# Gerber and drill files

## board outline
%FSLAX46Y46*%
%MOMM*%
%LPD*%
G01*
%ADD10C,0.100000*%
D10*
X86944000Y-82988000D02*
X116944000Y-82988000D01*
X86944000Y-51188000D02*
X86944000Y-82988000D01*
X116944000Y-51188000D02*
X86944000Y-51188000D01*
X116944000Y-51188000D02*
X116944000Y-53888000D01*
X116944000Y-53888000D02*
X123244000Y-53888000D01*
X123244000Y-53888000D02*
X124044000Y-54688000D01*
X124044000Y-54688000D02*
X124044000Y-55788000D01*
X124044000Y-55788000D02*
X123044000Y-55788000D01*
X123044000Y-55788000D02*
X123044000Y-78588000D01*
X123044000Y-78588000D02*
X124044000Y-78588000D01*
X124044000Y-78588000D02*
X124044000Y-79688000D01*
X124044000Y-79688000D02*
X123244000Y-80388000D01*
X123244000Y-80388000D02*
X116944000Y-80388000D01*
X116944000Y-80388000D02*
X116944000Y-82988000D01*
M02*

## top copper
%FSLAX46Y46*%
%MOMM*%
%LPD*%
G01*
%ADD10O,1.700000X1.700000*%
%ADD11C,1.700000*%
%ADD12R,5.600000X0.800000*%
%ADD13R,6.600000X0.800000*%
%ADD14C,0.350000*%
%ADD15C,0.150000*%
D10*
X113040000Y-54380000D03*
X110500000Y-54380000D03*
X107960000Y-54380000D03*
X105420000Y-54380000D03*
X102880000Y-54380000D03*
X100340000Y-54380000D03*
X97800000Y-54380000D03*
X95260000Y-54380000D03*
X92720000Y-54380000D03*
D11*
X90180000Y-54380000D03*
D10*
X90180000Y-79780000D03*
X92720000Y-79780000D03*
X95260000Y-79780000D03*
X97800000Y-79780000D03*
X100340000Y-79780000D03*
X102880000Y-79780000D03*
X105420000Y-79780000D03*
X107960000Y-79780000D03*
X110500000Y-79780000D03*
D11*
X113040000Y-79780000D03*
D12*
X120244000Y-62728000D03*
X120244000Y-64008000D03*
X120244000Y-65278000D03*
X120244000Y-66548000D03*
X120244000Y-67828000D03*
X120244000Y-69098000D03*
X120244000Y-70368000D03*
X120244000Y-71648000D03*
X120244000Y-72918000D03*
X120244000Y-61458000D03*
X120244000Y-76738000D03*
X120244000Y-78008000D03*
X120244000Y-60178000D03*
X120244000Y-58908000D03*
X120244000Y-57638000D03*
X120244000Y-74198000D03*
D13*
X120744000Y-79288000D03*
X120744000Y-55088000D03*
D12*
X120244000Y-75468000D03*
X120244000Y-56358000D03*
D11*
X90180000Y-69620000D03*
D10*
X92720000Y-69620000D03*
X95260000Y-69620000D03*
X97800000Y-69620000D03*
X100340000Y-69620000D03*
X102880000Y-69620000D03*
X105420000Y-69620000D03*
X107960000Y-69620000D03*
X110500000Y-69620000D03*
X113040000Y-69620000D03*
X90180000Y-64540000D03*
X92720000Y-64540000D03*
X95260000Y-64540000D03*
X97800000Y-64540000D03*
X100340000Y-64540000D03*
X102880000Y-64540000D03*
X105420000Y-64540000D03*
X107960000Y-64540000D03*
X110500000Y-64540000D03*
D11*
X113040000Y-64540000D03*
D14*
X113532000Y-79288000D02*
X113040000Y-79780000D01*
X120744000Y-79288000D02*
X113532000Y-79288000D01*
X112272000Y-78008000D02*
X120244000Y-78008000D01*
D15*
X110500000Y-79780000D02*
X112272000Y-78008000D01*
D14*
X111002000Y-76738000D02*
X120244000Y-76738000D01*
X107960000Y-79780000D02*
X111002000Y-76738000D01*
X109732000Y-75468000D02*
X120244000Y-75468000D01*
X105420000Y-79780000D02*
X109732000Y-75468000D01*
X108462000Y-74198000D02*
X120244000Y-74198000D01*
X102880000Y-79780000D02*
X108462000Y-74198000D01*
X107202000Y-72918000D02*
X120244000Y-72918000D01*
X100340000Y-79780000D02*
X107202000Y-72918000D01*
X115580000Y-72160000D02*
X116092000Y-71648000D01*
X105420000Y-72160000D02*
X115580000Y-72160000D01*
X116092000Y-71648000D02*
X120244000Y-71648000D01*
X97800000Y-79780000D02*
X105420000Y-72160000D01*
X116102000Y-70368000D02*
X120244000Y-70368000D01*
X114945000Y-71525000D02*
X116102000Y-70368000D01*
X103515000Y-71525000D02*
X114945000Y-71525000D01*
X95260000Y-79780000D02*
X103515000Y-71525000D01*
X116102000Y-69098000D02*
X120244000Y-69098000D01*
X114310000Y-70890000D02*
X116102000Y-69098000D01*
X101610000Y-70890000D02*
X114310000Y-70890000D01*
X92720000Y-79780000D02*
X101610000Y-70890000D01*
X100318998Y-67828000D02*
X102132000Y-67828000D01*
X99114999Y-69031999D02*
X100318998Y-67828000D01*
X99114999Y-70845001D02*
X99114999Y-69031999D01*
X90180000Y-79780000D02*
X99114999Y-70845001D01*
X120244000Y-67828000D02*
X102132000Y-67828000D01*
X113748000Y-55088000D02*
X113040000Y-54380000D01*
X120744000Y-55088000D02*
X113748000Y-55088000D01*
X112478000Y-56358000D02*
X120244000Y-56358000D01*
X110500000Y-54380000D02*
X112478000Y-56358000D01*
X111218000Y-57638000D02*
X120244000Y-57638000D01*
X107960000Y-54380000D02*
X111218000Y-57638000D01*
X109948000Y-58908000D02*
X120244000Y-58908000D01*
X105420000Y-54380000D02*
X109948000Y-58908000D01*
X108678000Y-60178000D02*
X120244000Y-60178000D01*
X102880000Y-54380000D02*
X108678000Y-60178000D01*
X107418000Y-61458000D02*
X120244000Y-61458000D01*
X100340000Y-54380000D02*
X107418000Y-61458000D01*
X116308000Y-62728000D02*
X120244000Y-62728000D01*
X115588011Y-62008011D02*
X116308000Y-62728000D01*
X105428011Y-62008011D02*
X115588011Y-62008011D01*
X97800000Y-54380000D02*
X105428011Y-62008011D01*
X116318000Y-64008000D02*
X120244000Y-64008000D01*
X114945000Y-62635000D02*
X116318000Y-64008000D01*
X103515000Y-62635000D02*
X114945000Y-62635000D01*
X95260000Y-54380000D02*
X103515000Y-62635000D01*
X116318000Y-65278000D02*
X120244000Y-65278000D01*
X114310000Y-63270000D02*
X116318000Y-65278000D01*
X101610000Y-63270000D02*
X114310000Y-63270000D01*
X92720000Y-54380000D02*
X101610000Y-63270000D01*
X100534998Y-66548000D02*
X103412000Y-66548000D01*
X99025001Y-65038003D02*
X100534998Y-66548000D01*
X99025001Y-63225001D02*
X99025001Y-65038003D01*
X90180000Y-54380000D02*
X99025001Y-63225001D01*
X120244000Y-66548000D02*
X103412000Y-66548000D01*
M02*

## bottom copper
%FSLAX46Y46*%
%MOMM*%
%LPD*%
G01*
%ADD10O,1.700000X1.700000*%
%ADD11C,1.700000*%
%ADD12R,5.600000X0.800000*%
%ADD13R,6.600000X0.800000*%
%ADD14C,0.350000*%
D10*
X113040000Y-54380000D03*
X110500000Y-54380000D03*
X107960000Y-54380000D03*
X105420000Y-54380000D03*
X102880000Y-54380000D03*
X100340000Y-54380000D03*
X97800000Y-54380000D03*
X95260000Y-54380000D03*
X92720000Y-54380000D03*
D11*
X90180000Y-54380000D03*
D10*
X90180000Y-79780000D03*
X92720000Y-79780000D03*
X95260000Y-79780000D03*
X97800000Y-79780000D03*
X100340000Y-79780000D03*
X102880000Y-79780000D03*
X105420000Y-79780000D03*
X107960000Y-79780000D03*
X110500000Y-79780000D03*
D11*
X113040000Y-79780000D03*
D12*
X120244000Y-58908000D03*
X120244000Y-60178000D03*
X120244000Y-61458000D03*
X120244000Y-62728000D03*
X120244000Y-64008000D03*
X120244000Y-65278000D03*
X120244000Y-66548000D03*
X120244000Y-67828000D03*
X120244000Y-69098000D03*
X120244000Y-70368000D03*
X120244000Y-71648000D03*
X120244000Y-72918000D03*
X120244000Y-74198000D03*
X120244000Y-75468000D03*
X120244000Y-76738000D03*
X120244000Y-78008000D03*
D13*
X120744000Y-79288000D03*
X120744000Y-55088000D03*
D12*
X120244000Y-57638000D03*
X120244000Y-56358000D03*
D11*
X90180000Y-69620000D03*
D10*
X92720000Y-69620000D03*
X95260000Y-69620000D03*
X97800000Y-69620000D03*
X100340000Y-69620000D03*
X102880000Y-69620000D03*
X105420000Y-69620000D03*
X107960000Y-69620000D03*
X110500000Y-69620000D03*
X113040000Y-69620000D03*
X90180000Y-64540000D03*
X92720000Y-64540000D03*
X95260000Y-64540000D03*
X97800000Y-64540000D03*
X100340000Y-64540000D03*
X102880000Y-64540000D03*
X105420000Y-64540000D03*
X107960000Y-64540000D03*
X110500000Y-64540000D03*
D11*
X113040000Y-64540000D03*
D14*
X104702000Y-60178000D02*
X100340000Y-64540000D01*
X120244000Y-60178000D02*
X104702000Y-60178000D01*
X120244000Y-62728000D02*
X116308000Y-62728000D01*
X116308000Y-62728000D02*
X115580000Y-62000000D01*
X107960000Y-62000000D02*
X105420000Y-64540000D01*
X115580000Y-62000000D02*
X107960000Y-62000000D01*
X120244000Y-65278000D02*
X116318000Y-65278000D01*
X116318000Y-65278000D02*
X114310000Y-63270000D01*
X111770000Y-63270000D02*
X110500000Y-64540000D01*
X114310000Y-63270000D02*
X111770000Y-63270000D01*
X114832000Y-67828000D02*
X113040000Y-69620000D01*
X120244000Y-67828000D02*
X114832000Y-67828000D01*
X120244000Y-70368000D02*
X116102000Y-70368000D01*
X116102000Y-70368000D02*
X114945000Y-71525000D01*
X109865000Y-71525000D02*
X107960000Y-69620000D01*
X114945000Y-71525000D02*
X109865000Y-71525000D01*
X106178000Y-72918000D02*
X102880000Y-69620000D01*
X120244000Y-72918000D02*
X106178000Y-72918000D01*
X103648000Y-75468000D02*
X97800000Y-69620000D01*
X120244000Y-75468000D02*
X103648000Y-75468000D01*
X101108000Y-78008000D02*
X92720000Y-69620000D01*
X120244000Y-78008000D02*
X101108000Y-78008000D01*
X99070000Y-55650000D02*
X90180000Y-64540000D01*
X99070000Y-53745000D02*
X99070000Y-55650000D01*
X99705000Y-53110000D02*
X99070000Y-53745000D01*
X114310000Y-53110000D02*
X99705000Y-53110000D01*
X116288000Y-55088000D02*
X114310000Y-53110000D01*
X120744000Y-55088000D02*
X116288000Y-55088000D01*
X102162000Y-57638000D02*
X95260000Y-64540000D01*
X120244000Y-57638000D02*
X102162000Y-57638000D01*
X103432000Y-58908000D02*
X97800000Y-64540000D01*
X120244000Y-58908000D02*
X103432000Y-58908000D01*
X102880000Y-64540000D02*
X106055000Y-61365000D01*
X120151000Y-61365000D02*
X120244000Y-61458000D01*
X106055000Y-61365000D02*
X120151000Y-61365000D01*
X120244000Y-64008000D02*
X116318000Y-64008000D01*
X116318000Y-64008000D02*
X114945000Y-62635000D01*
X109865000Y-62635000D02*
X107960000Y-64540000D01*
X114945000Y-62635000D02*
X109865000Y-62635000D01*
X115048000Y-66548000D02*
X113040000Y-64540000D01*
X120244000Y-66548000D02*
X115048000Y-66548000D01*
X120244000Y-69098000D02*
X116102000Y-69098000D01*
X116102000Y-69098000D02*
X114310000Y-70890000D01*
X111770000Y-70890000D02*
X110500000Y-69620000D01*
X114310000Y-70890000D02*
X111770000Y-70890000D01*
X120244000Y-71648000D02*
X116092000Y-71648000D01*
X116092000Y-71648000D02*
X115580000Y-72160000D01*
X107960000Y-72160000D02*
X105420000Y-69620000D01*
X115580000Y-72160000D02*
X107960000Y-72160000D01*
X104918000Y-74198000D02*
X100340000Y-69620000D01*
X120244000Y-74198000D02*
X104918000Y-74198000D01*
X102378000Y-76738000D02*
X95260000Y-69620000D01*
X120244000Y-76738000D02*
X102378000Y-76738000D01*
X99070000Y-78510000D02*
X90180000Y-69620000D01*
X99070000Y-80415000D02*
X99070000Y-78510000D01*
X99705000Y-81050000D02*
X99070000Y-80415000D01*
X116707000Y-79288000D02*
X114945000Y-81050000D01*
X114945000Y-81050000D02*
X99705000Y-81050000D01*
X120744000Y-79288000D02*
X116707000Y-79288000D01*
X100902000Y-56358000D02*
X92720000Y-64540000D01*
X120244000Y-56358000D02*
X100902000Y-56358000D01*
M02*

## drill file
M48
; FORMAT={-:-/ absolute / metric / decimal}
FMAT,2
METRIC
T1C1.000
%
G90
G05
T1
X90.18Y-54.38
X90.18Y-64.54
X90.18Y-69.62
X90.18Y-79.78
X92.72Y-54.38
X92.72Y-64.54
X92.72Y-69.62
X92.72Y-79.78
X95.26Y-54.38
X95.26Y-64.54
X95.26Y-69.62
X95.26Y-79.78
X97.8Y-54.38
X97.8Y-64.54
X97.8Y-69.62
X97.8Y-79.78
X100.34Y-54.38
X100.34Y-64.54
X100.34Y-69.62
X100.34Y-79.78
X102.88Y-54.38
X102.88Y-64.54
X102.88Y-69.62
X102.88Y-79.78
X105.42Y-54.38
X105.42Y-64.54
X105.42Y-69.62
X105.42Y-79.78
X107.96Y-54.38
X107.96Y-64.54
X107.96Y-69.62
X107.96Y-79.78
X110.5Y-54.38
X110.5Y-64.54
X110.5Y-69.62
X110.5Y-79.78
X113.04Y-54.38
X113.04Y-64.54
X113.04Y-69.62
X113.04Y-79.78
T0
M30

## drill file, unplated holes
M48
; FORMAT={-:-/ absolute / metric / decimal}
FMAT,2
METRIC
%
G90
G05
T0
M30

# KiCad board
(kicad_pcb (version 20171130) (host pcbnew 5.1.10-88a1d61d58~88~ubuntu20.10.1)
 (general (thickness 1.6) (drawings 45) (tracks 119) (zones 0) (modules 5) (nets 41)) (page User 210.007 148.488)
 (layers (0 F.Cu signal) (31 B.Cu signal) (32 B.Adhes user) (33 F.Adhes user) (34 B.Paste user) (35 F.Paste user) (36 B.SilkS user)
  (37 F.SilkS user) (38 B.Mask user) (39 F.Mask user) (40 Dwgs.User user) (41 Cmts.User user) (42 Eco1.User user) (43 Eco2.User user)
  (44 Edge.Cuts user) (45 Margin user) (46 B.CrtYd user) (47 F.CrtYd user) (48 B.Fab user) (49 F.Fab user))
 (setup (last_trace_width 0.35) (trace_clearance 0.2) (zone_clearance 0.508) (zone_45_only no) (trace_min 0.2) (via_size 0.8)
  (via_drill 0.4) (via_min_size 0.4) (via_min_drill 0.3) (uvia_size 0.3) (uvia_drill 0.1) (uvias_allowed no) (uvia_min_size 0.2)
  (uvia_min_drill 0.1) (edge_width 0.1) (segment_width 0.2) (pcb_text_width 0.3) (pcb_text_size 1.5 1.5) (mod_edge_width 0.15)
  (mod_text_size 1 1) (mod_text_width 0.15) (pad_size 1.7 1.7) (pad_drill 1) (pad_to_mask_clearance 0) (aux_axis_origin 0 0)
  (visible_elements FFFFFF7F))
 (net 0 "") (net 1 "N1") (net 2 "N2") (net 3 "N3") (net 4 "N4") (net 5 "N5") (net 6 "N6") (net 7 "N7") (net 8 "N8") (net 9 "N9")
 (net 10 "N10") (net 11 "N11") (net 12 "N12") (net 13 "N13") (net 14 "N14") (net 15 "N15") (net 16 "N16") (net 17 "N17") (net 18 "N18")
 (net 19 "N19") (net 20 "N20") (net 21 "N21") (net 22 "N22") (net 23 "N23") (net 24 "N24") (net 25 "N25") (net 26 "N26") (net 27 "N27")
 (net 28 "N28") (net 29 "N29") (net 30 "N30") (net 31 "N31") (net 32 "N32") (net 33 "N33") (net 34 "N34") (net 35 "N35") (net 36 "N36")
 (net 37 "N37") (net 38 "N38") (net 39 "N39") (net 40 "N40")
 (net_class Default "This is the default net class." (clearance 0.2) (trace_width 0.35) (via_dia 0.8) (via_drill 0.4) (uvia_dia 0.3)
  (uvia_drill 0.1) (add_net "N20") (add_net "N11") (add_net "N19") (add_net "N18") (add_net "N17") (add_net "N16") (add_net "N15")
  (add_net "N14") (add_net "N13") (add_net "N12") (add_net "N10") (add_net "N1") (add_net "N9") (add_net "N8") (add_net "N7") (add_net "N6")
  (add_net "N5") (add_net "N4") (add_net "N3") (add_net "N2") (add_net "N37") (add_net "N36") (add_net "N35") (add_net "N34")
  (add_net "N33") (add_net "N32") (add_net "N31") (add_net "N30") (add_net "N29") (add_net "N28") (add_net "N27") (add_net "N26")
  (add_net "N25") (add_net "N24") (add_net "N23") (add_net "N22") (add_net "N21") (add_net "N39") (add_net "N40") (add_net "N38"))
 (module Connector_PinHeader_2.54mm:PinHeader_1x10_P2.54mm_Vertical (layer F.Cu) (at 90.18 54.38 90)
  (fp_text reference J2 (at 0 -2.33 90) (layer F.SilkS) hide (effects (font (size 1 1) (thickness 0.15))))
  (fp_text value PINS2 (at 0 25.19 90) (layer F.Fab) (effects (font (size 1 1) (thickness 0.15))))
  (pad 10 thru_hole oval (at 0 22.86 90) (size 1.7 1.7) (drill 1) (layers *.Cu *.Mask) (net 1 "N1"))
  (pad 9 thru_hole oval (at 0 20.32 90) (size 1.7 1.7) (drill 1) (layers *.Cu *.Mask) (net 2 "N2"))
  (pad 8 thru_hole oval (at 0 17.78 90) (size 1.7 1.7) (drill 1) (layers *.Cu *.Mask) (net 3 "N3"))
  (pad 7 thru_hole oval (at 0 15.24 90) (size 1.7 1.7) (drill 1) (layers *.Cu *.Mask) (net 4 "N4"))
  (pad 6 thru_hole oval (at 0 12.7 90) (size 1.7 1.7) (drill 1) (layers *.Cu *.Mask) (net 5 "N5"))
  (pad 5 thru_hole oval (at 0 10.16 90) (size 1.7 1.7) (drill 1) (layers *.Cu *.Mask) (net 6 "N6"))
  (pad 4 thru_hole oval (at 0 7.62 90) (size 1.7 1.7) (drill 1) (layers *.Cu *.Mask) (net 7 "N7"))
  (pad 3 thru_hole oval (at 0 5.08 90) (size 1.7 1.7) (drill 1) (layers *.Cu *.Mask) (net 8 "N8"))
  (pad 2 thru_hole oval (at 0 2.54 90) (size 1.7 1.7) (drill 1) (layers *.Cu *.Mask) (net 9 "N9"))
  (pad 1 thru_hole circle (at 0 0 90) (size 1.7 1.7) (drill 1) (layers *.Cu *.Mask) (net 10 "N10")))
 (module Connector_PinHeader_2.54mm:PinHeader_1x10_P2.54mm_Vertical (layer F.Cu) (at 113.04 79.78 270)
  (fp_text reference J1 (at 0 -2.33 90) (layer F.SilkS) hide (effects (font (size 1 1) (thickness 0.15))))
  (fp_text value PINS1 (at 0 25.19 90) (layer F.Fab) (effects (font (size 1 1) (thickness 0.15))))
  (pad 10 thru_hole oval (at 0 22.86 270) (size 1.7 1.7) (drill 1) (layers *.Cu *.Mask) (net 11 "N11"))
  (pad 9 thru_hole oval (at 0 20.32 270) (size 1.7 1.7) (drill 1) (layers *.Cu *.Mask) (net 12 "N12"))
  (pad 8 thru_hole oval (at 0 17.78 270) (size 1.7 1.7) (drill 1) (layers *.Cu *.Mask) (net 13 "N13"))
  (pad 7 thru_hole oval (at 0 15.24 270) (size 1.7 1.7) (drill 1) (layers *.Cu *.Mask) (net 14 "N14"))
  (pad 6 thru_hole oval (at 0 12.7 270) (size 1.7 1.7) (drill 1) (layers *.Cu *.Mask) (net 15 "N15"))
  (pad 5 thru_hole oval (at 0 10.16 270) (size 1.7 1.7) (drill 1) (layers *.Cu *.Mask) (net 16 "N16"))
  (pad 4 thru_hole oval (at 0 7.62 270) (size 1.7 1.7) (drill 1) (layers *.Cu *.Mask) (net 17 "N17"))
  (pad 3 thru_hole oval (at 0 5.08 270) (size 1.7 1.7) (drill 1) (layers *.Cu *.Mask) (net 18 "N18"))
  (pad 2 thru_hole oval (at 0 2.54 270) (size 1.7 1.7) (drill 1) (layers *.Cu *.Mask) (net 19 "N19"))
  (pad 1 thru_hole circle (at 0 0 270) (size 1.7 1.7) (drill 1) (layers *.Cu *.Mask) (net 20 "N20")))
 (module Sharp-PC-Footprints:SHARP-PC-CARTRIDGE (layer F.Cu) (at 116.944 51.188)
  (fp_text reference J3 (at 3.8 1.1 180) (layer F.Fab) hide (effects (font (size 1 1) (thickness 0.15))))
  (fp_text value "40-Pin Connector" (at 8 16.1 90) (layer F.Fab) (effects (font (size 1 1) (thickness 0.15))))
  (fp_line (start 0 0) (end 0 2.7) (layer Edge.Cuts) (width 0.1))
  (fp_line (start 0 2.7) (end 6.3 2.7) (layer Edge.Cuts) (width 0.1))
  (fp_line (start 6.3 2.7) (end 7.1 3.5) (layer Edge.Cuts) (width 0.1))
  (fp_line (start 7.1 3.5) (end 7.1 4.6) (layer Edge.Cuts) (width 0.1))
  (fp_line (start 7.1 4.6) (end 6.1 4.6) (layer Edge.Cuts) (width 0.1))
  (fp_line (start 6.1 4.6) (end 6.1 27.4) (layer Edge.Cuts) (width 0.1))
  (fp_line (start 6.1 27.4) (end 7.1 27.4) (layer Edge.Cuts) (width 0.1))
  (fp_line (start 7.1 27.4) (end 7.1 28.5) (layer Edge.Cuts) (width 0.1))
  (fp_line (start 7.1 28.5) (end 6.3 29.2) (layer Edge.Cuts) (width 0.1))
  (fp_line (start 6.3 29.2) (end 0 29.2) (layer Edge.Cuts) (width 0.1))
  (fp_line (start 0 29.2) (end 0 31.8) (layer Edge.Cuts) (width 0.1))
  (pad 37 smd rect (at 3.3 7.72 180) (size 5.6 0.8) (layers B.Cu B.Paste B.Mask) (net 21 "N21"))
  (pad 36 smd rect (at 3.3 8.99 180) (size 5.6 0.8) (layers B.Cu B.Paste B.Mask) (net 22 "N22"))
  (pad 35 smd rect (at 3.3 10.27 180) (size 5.6 0.8) (layers B.Cu B.Paste B.Mask) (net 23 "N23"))
  (pad 34 smd rect (at 3.3 11.54 180) (size 5.6 0.8) (layers B.Cu B.Paste B.Mask) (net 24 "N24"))
  (pad 33 smd rect (at 3.3 12.82 180) (size 5.6 0.8) (layers B.Cu B.Paste B.Mask) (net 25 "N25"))
  (pad 32 smd rect (at 3.3 14.09 180) (size 5.6 0.8) (layers B.Cu B.Paste B.Mask) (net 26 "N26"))
  (pad 31 smd rect (at 3.3 15.36 180) (size 5.6 0.8) (layers B.Cu B.Paste B.Mask) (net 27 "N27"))
  (pad 30 smd rect (at 3.3 16.64 180) (size 5.6 0.8) (layers B.Cu B.Paste B.Mask) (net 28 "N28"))
  (pad 29 smd rect (at 3.3 17.91 180) (size 5.6 0.8) (layers B.Cu B.Paste B.Mask) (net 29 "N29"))
  (pad 28 smd rect (at 3.3 19.18 180) (size 5.6 0.8) (layers B.Cu B.Paste B.Mask) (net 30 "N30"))
  (pad 27 smd rect (at 3.3 20.46 180) (size 5.6 0.8) (layers B.Cu B.Paste B.Mask) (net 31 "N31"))
  (pad 26 smd rect (at 3.3 21.73 180) (size 5.6 0.8) (layers B.Cu B.Paste B.Mask) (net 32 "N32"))
  (pad 25 smd rect (at 3.3 23.01 180) (size 5.6 0.8) (layers B.Cu B.Paste B.Mask) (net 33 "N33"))
  (pad 24 smd rect (at 3.3 24.28 180) (size 5.6 0.8) (layers B.Cu B.Paste B.Mask) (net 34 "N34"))
  (pad 23 smd rect (at 3.3 25.55 180) (size 5.6 0.8) (layers B.Cu B.Paste B.Mask) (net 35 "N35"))
  (pad 22 smd rect (at 3.3 26.82 180) (size 5.6 0.8) (layers B.Cu B.Paste B.Mask) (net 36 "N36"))
  (pad 14 smd rect (at 3.3 11.54 180) (size 5.6 0.8) (layers F.Cu F.Paste F.Mask) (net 7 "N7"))
  (pad 13 smd rect (at 3.3 12.82 180) (size 5.6 0.8) (layers F.Cu F.Paste F.Mask) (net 8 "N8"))
  (pad 12 smd rect (at 3.3 14.09 180) (size 5.6 0.8) (layers F.Cu F.Paste F.Mask) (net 9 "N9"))
  (pad 11 smd rect (at 3.3 15.36 180) (size 5.6 0.8) (layers F.Cu F.Paste F.Mask) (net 10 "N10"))
  (pad 10 smd rect (at 3.3 16.64 180) (size 5.6 0.8) (layers F.Cu F.Paste F.Mask) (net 11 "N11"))
  (pad 9 smd rect (at 3.3 17.91 180) (size 5.6 0.8) (layers F.Cu F.Paste F.Mask) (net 12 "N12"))
  (pad 8 smd rect (at 3.3 19.18 180) (size 5.6 0.8) (layers F.Cu F.Paste F.Mask) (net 13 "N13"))
  (pad 7 smd rect (at 3.3 20.46 180) (size 5.6 0.8) (layers F.Cu F.Paste F.Mask) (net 14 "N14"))
  (pad 6 smd rect (at 3.3 21.73 180) (size 5.6 0.8) (layers F.Cu F.Paste F.Mask) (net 15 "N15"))
  (pad 21 smd rect (at 3.8 28.1 180) (size 6.6 0.8) (layers B.Cu B.Paste B.Mask) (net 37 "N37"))
  (pad 40 smd rect (at 3.8 3.9 180) (size 6.6 0.8) (layers B.Cu B.Paste B.Mask) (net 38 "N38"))
  (pad 15 smd rect (at 3.3 10.27 180) (size 5.6 0.8) (layers F.Cu F.Paste F.Mask) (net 6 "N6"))
  (pad 38 smd rect (at 3.3 6.45 180) (size 5.6 0.8) (layers B.Cu B.Paste B.Mask) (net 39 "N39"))
  (pad 3 smd rect (at 3.3 25.55 180) (size 5.6 0.8) (layers F.Cu F.Paste F.Mask) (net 18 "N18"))
  (pad 2 smd rect (at 3.3 26.82 180) (size 5.6 0.8) (layers F.Cu F.Paste F.Mask) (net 19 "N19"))
  (pad 39 smd rect (at 3.3 5.17 180) (size 5.6 0.8) (layers B.Cu B.Paste B.Mask) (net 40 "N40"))
  (pad 16 smd rect (at 3.3 8.99 180) (size 5.6 0.8) (layers F.Cu F.Paste F.Mask) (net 5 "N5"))
  (pad 17 smd rect (at 3.3 7.72 180) (size 5.6 0.8) (layers F.Cu F.Paste F.Mask) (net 4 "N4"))
  (pad 18 smd rect (at 3.3 6.45 180) (size 5.6 0.8) (layers F.Cu F.Paste F.Mask) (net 3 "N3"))
  (pad 5 smd rect (at 3.3 23.01 180) (size 5.6 0.8) (layers F.Cu F.Paste F.Mask) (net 16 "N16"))
  (pad 1 smd rect (at 3.8 28.1 180) (size 6.6 0.8) (layers F.Cu F.Paste F.Mask) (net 20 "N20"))
  (pad 20 smd rect (at 3.8 3.9 180) (size 6.6 0.8) (layers F.Cu F.Paste F.Mask) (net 1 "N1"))
  (pad 4 smd rect (at 3.3 24.28 180) (size 5.6 0.8) (layers F.Cu F.Paste F.Mask) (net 17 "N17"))
  (pad 19 smd rect (at 3.3 5.17 180) (size 5.6 0.8) (layers F.Cu F.Paste F.Mask) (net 2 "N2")))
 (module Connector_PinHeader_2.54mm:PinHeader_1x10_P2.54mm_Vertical (layer F.Cu) (at 90.18 69.62 90)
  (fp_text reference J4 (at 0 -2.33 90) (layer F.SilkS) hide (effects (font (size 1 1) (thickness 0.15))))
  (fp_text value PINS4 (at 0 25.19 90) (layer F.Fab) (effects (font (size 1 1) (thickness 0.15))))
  (pad 1 thru_hole circle (at 0 0 90) (size 1.7 1.7) (drill 1) (layers *.Cu *.Mask) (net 37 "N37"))
  (pad 2 thru_hole oval (at 0 2.54 90) (size 1.7 1.7) (drill 1) (layers *.Cu *.Mask) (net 36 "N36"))
  (pad 3 thru_hole oval (at 0 5.08 90) (size 1.7 1.7) (drill 1) (layers *.Cu *.Mask) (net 35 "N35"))
  (pad 4 thru_hole oval (at 0 7.62 90) (size 1.7 1.7) (drill 1) (layers *.Cu *.Mask) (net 34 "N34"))
  (pad 5 thru_hole oval (at 0 10.16 90) (size 1.7 1.7) (drill 1) (layers *.Cu *.Mask) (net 33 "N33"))
  (pad 6 thru_hole oval (at 0 12.7 90) (size 1.7 1.7) (drill 1) (layers *.Cu *.Mask) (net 32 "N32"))
  (pad 7 thru_hole oval (at 0 15.24 90) (size 1.7 1.7) (drill 1) (layers *.Cu *.Mask) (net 31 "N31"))
  (pad 8 thru_hole oval (at 0 17.78 90) (size 1.7 1.7) (drill 1) (layers *.Cu *.Mask) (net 30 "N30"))
  (pad 9 thru_hole oval (at 0 20.32 90) (size 1.7 1.7) (drill 1) (layers *.Cu *.Mask) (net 29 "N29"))
  (pad 10 thru_hole oval (at 0 22.86 90) (size 1.7 1.7) (drill 1) (layers *.Cu *.Mask) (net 28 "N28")))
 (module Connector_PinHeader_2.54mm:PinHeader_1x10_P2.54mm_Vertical (layer F.Cu) (at 113.04 64.54 270)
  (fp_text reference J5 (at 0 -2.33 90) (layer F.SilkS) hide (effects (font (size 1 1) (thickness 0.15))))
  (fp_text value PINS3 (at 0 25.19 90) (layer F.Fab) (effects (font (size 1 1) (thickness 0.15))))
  (pad 10 thru_hole oval (at 0 22.86 270) (size 1.7 1.7) (drill 1) (layers *.Cu *.Mask) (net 38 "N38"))
  (pad 9 thru_hole oval (at 0 20.32 270) (size 1.7 1.7) (drill 1) (layers *.Cu *.Mask) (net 40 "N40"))
  (pad 8 thru_hole oval (at 0 17.78 270) (size 1.7 1.7) (drill 1) (layers *.Cu *.Mask) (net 39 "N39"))
  (pad 7 thru_hole oval (at 0 15.24 270) (size 1.7 1.7) (drill 1) (layers *.Cu *.Mask) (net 21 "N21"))
  (pad 6 thru_hole oval (at 0 12.7 270) (size 1.7 1.7) (drill 1) (layers *.Cu *.Mask) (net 22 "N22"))
  (pad 5 thru_hole oval (at 0 10.16 270) (size 1.7 1.7) (drill 1) (layers *.Cu *.Mask) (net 23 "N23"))
  (pad 4 thru_hole oval (at 0 7.62 270) (size 1.7 1.7) (drill 1) (layers *.Cu *.Mask) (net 24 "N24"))
  (pad 3 thru_hole oval (at 0 5.08 270) (size 1.7 1.7) (drill 1) (layers *.Cu *.Mask) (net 25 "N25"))
  (pad 2 thru_hole oval (at 0 2.54 270) (size 1.7 1.7) (drill 1) (layers *.Cu *.Mask) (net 26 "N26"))
  (pad 1 thru_hole circle (at 0 0 270) (size 1.7 1.7) (drill 1) (layers *.Cu *.Mask) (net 27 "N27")))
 (gr_line (start 86.944 82.988) (end 116.944 82.988) (layer Edge.Cuts) (width 0.1))
 (gr_line (start 86.944 51.188) (end 86.944 82.988) (layer Edge.Cuts) (width 0.1))
 (gr_line (start 116.944 51.188) (end 86.944 51.188) (layer Edge.Cuts) (width 0.1))
 (segment (start 113.532 79.288) (end 113.04 79.78) (width 0.35) (layer F.Cu) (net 20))
 (segment (start 120.744 79.288) (end 113.532 79.288) (width 0.35) (layer F.Cu) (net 20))
 (segment (start 112.272 78.008) (end 120.244 78.008) (width 0.35) (layer F.Cu) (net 19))
 (segment (start 110.5 79.78) (end 112.272 78.008) (width 0.15) (layer F.Cu) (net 19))
 (segment (start 111.002 76.738) (end 120.244 76.738) (width 0.35) (layer F.Cu) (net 18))
 (segment (start 107.96 79.78) (end 111.002 76.738) (width 0.35) (layer F.Cu) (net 18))
 (segment (start 109.732 75.468) (end 120.244 75.468) (width 0.35) (layer F.Cu) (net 17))
 (segment (start 105.42 79.78) (end 109.732 75.468) (width 0.35) (layer F.Cu) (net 17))
 (segment (start 108.462 74.198) (end 120.244 74.198) (width 0.35) (layer F.Cu) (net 16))
 (segment (start 102.88 79.78) (end 108.462 74.198) (width 0.35) (layer F.Cu) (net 16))
 (segment (start 107.202 72.918) (end 120.244 72.918) (width 0.35) (layer F.Cu) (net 15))
 (segment (start 100.34 79.78) (end 107.202 72.918) (width 0.35) (layer F.Cu) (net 15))
 (segment (start 115.58 72.16) (end 116.092 71.648) (width 0.35) (layer F.Cu) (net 14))
 (segment (start 105.42 72.16) (end 115.58 72.16) (width 0.35) (layer F.Cu) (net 14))
 (segment (start 116.092 71.648) (end 120.244 71.648) (width 0.35) (layer F.Cu) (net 14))
 (segment (start 97.8 79.78) (end 105.42 72.16) (width 0.35) (layer F.Cu) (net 14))
 (segment (start 116.102 70.368) (end 120.244 70.368) (width 0.35) (layer F.Cu) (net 13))
 (segment (start 114.945 71.525) (end 116.102 70.368) (width 0.35) (layer F.Cu) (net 13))
 (segment (start 103.515 71.525) (end 114.945 71.525) (width 0.35) (layer F.Cu) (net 13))
 (segment (start 95.26 79.78) (end 103.515 71.525) (width 0.35) (layer F.Cu) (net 13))
 (segment (start 116.102 69.098) (end 120.244 69.098) (width 0.35) (layer F.Cu) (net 12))
 (segment (start 114.31 70.89) (end 116.102 69.098) (width 0.35) (layer F.Cu) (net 12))
 (segment (start 101.61 70.89) (end 114.31 70.89) (width 0.35) (layer F.Cu) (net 12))
 (segment (start 92.72 79.78) (end 101.61 70.89) (width 0.35) (layer F.Cu) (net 12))
 (segment (start 100.318998 67.828) (end 102.132 67.828) (width 0.35) (layer F.Cu) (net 11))
 (segment (start 99.114999 69.031999) (end 100.318998 67.828) (width 0.35) (layer F.Cu) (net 11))
 (segment (start 99.114999 70.845001) (end 99.114999 69.031999) (width 0.35) (layer F.Cu) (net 11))
 (segment (start 90.18 79.78) (end 99.114999 70.845001) (width 0.35) (layer F.Cu) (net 11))
 (segment (start 120.244 67.828) (end 102.132 67.828) (width 0.35) (layer F.Cu) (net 11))
 (segment (start 113.748 55.088) (end 113.04 54.38) (width 0.35) (layer F.Cu) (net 1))
 (segment (start 120.744 55.088) (end 113.748 55.088) (width 0.35) (layer F.Cu) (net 1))
 (segment (start 112.478 56.358) (end 120.244 56.358) (width 0.35) (layer F.Cu) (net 2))
 (segment (start 110.5 54.38) (end 112.478 56.358) (width 0.35) (layer F.Cu) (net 2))
 (segment (start 111.218 57.638) (end 120.244 57.638) (width 0.35) (layer F.Cu) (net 3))
 (segment (start 107.96 54.38) (end 111.218 57.638) (width 0.35) (layer F.Cu) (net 3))
 (segment (start 109.948 58.908) (end 120.244 58.908) (width 0.35) (layer F.Cu) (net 4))
 (segment (start 105.42 54.38) (end 109.948 58.908) (width 0.35) (layer F.Cu) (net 4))
 (segment (start 108.678 60.178) (end 120.244 60.178) (width 0.35) (layer F.Cu) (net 5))
 (segment (start 102.88 54.38) (end 108.678 60.178) (width 0.35) (layer F.Cu) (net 5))
 (segment (start 107.418 61.458) (end 120.244 61.458) (width 0.35) (layer F.Cu) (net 6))
 (segment (start 100.34 54.38) (end 107.418 61.458) (width 0.35) (layer F.Cu) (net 6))
 (segment (start 116.308 62.728) (end 120.244 62.728) (width 0.35) (layer F.Cu) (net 7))
 (segment (start 115.588011 62.008011) (end 116.308 62.728) (width 0.35) (layer F.Cu) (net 7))
 (segment (start 105.428011 62.008011) (end 115.588011 62.008011) (width 0.35) (layer F.Cu) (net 7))
 (segment (start 97.8 54.38) (end 105.428011 62.008011) (width 0.35) (layer F.Cu) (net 7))
 (segment (start 116.318 64.008) (end 120.244 64.008) (width 0.35) (layer F.Cu) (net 8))
 (segment (start 114.945 62.635) (end 116.318 64.008) (width 0.35) (layer F.Cu) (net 8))
 (segment (start 103.515 62.635) (end 114.945 62.635) (width 0.35) (layer F.Cu) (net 8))
 (segment (start 95.26 54.38) (end 103.515 62.635) (width 0.35) (layer F.Cu) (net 8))
 (segment (start 116.318 65.278) (end 120.244 65.278) (width 0.35) (layer F.Cu) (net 9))
 (segment (start 114.31 63.27) (end 116.318 65.278) (width 0.35) (layer F.Cu) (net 9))
 (segment (start 101.61 63.27) (end 114.31 63.27) (width 0.35) (layer F.Cu) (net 9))
 (segment (start 92.72 54.38) (end 101.61 63.27) (width 0.35) (layer F.Cu) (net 9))
 (segment (start 100.534998 66.548) (end 103.412 66.548) (width 0.35) (layer F.Cu) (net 10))
 (segment (start 99.025001 65.038003) (end 100.534998 66.548) (width 0.35) (layer F.Cu) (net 10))
 (segment (start 99.025001 63.225001) (end 99.025001 65.038003) (width 0.35) (layer F.Cu) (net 10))
 (segment (start 90.18 54.38) (end 99.025001 63.225001) (width 0.35) (layer F.Cu) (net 10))
 (segment (start 120.244 66.548) (end 103.412 66.548) (width 0.35) (layer F.Cu) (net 10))
 (segment (start 104.702 60.178) (end 100.34 64.54) (width 0.35) (layer B.Cu) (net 22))
 (segment (start 120.244 60.178) (end 104.702 60.178) (width 0.35) (layer B.Cu) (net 22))
 (segment (start 120.244 62.728) (end 116.308 62.728) (width 0.35) (layer B.Cu) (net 24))
 (segment (start 116.308 62.728) (end 115.58 62) (width 0.35) (layer B.Cu) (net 24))
 (segment (start 107.96 62) (end 105.42 64.54) (width 0.35) (layer B.Cu) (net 24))
 (segment (start 115.58 62) (end 107.96 62) (width 0.35) (layer B.Cu) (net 24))
 (segment (start 120.244 65.278) (end 116.318 65.278) (width 0.35) (layer B.Cu) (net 26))
 (segment (start 116.318 65.278) (end 114.31 63.27) (width 0.35) (layer B.Cu) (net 26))
 (segment (start 111.77 63.27) (end 110.5 64.54) (width 0.35) (layer B.Cu) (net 26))
 (segment (start 114.31 63.27) (end 111.77 63.27) (width 0.35) (layer B.Cu) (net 26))
 (segment (start 114.832 67.828) (end 113.04 69.62) (width 0.35) (layer B.Cu) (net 28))
 (segment (start 120.244 67.828) (end 114.832 67.828) (width 0.35) (layer B.Cu) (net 28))
 (segment (start 120.244 70.368) (end 116.102 70.368) (width 0.35) (layer B.Cu) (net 30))
 (segment (start 116.102 70.368) (end 114.945 71.525) (width 0.35) (layer B.Cu) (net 30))
 (segment (start 109.865 71.525) (end 107.96 69.62) (width 0.35) (layer B.Cu) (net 30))
 (segment (start 114.945 71.525) (end 109.865 71.525) (width 0.35) (layer B.Cu) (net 30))
 (segment (start 106.178 72.918) (end 102.88 69.62) (width 0.35) (layer B.Cu) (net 32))
 (segment (start 120.244 72.918) (end 106.178 72.918) (width 0.35) (layer B.Cu) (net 32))
 (segment (start 103.648 75.468) (end 97.8 69.62) (width 0.35) (layer B.Cu) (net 34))
 (segment (start 120.244 75.468) (end 103.648 75.468) (width 0.35) (layer B.Cu) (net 34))
 (segment (start 101.108 78.008) (end 92.72 69.62) (width 0.35) (layer B.Cu) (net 36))
 (segment (start 120.244 78.008) (end 101.108 78.008) (width 0.35) (layer B.Cu) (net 36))
 (segment (start 99.07 55.65) (end 90.18 64.54) (width 0.35) (layer B.Cu) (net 38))
 (segment (start 99.07 53.745) (end 99.07 55.65) (width 0.35) (layer B.Cu) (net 38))
 (segment (start 99.705 53.11) (end 99.07 53.745) (width 0.35) (layer B.Cu) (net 38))
 (segment (start 114.31 53.11) (end 99.705 53.11) (width 0.35) (layer B.Cu) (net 38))
 (segment (start 116.288 55.088) (end 114.31 53.11) (width 0.35) (layer B.Cu) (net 38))
 (segment (start 120.744 55.088) (end 116.288 55.088) (width 0.35) (layer B.Cu) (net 38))
 (segment (start 102.162 57.638) (end 95.26 64.54) (width 0.35) (layer B.Cu) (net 39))
 (segment (start 120.244 57.638) (end 102.162 57.638) (width 0.35) (layer B.Cu) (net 39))
 (segment (start 103.432 58.908) (end 97.8 64.54) (width 0.35) (layer B.Cu) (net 21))
 (segment (start 120.244 58.908) (end 103.432 58.908) (width 0.35) (layer B.Cu) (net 21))
 (segment (start 102.88 64.54) (end 106.055 61.365) (width 0.35) (layer B.Cu) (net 23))
 (segment (start 120.151 61.365) (end 120.244 61.458) (width 0.35) (layer B.Cu) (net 23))
 (segment (start 106.055 61.365) (end 120.151 61.365) (width 0.35) (layer B.Cu) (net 23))
 (segment (start 120.244 64.008) (end 116.318 64.008) (width 0.35) (layer B.Cu) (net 25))
 (segment (start 116.318 64.008) (end 114.945 62.635) (width 0.35) (layer B.Cu) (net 25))
 (segment (start 109.865 62.635) (end 107.96 64.54) (width 0.35) (layer B.Cu) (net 25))
 (segment (start 114.945 62.635) (end 109.865 62.635) (width 0.35) (layer B.Cu) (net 25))
 (segment (start 115.048 66.548) (end 113.04 64.54) (width 0.35) (layer B.Cu) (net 27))
 (segment (start 120.244 66.548) (end 115.048 66.548) (width 0.35) (layer B.Cu) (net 27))
 (segment (start 120.244 69.098) (end 116.102 69.098) (width 0.35) (layer B.Cu) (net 29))
 (segment (start 116.102 69.098) (end 114.31 70.89) (width 0.35) (layer B.Cu) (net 29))
 (segment (start 111.77 70.89) (end 110.5 69.62) (width 0.35) (layer B.Cu) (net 29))
 (segment (start 114.31 70.89) (end 111.77 70.89) (width 0.35) (layer B.Cu) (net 29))
 (segment (start 120.244 71.648) (end 116.092 71.648) (width 0.35) (layer B.Cu) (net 31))
 (segment (start 116.092 71.648) (end 115.58 72.16) (width 0.35) (layer B.Cu) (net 31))
 (segment (start 107.96 72.16) (end 105.42 69.62) (width 0.35) (layer B.Cu) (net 31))
 (segment (start 115.58 72.16) (end 107.96 72.16) (width 0.35) (layer B.Cu) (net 31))
 (segment (start 104.918 74.198) (end 100.34 69.62) (width 0.35) (layer B.Cu) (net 33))
 (segment (start 120.244 74.198) (end 104.918 74.198) (width 0.35) (layer B.Cu) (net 33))
 (segment (start 102.378 76.738) (end 95.26 69.62) (width 0.35) (layer B.Cu) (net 35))
 (segment (start 120.244 76.738) (end 102.378 76.738) (width 0.35) (layer B.Cu) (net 35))
 (segment (start 99.07 78.51) (end 90.18 69.62) (width 0.35) (layer B.Cu) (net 37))
 (segment (start 99.07 80.415) (end 99.07 78.51) (width 0.35) (layer B.Cu) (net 37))
 (segment (start 99.705 81.05) (end 99.07 80.415) (width 0.35) (layer B.Cu) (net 37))
 (segment (start 116.707 79.288) (end 114.945 81.05) (width 0.35) (layer B.Cu) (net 37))
 (segment (start 114.945 81.05) (end 99.705 81.05) (width 0.35) (layer B.Cu) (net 37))
 (segment (start 120.744 79.288) (end 116.707 79.288) (width 0.35) (layer B.Cu) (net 37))
 (segment (start 100.902 56.358) (end 92.72 64.54) (width 0.35) (layer B.Cu) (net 40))
 (segment (start 120.244 56.358) (end 100.902 56.358) (width 0.35) (layer B.Cu) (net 40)))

